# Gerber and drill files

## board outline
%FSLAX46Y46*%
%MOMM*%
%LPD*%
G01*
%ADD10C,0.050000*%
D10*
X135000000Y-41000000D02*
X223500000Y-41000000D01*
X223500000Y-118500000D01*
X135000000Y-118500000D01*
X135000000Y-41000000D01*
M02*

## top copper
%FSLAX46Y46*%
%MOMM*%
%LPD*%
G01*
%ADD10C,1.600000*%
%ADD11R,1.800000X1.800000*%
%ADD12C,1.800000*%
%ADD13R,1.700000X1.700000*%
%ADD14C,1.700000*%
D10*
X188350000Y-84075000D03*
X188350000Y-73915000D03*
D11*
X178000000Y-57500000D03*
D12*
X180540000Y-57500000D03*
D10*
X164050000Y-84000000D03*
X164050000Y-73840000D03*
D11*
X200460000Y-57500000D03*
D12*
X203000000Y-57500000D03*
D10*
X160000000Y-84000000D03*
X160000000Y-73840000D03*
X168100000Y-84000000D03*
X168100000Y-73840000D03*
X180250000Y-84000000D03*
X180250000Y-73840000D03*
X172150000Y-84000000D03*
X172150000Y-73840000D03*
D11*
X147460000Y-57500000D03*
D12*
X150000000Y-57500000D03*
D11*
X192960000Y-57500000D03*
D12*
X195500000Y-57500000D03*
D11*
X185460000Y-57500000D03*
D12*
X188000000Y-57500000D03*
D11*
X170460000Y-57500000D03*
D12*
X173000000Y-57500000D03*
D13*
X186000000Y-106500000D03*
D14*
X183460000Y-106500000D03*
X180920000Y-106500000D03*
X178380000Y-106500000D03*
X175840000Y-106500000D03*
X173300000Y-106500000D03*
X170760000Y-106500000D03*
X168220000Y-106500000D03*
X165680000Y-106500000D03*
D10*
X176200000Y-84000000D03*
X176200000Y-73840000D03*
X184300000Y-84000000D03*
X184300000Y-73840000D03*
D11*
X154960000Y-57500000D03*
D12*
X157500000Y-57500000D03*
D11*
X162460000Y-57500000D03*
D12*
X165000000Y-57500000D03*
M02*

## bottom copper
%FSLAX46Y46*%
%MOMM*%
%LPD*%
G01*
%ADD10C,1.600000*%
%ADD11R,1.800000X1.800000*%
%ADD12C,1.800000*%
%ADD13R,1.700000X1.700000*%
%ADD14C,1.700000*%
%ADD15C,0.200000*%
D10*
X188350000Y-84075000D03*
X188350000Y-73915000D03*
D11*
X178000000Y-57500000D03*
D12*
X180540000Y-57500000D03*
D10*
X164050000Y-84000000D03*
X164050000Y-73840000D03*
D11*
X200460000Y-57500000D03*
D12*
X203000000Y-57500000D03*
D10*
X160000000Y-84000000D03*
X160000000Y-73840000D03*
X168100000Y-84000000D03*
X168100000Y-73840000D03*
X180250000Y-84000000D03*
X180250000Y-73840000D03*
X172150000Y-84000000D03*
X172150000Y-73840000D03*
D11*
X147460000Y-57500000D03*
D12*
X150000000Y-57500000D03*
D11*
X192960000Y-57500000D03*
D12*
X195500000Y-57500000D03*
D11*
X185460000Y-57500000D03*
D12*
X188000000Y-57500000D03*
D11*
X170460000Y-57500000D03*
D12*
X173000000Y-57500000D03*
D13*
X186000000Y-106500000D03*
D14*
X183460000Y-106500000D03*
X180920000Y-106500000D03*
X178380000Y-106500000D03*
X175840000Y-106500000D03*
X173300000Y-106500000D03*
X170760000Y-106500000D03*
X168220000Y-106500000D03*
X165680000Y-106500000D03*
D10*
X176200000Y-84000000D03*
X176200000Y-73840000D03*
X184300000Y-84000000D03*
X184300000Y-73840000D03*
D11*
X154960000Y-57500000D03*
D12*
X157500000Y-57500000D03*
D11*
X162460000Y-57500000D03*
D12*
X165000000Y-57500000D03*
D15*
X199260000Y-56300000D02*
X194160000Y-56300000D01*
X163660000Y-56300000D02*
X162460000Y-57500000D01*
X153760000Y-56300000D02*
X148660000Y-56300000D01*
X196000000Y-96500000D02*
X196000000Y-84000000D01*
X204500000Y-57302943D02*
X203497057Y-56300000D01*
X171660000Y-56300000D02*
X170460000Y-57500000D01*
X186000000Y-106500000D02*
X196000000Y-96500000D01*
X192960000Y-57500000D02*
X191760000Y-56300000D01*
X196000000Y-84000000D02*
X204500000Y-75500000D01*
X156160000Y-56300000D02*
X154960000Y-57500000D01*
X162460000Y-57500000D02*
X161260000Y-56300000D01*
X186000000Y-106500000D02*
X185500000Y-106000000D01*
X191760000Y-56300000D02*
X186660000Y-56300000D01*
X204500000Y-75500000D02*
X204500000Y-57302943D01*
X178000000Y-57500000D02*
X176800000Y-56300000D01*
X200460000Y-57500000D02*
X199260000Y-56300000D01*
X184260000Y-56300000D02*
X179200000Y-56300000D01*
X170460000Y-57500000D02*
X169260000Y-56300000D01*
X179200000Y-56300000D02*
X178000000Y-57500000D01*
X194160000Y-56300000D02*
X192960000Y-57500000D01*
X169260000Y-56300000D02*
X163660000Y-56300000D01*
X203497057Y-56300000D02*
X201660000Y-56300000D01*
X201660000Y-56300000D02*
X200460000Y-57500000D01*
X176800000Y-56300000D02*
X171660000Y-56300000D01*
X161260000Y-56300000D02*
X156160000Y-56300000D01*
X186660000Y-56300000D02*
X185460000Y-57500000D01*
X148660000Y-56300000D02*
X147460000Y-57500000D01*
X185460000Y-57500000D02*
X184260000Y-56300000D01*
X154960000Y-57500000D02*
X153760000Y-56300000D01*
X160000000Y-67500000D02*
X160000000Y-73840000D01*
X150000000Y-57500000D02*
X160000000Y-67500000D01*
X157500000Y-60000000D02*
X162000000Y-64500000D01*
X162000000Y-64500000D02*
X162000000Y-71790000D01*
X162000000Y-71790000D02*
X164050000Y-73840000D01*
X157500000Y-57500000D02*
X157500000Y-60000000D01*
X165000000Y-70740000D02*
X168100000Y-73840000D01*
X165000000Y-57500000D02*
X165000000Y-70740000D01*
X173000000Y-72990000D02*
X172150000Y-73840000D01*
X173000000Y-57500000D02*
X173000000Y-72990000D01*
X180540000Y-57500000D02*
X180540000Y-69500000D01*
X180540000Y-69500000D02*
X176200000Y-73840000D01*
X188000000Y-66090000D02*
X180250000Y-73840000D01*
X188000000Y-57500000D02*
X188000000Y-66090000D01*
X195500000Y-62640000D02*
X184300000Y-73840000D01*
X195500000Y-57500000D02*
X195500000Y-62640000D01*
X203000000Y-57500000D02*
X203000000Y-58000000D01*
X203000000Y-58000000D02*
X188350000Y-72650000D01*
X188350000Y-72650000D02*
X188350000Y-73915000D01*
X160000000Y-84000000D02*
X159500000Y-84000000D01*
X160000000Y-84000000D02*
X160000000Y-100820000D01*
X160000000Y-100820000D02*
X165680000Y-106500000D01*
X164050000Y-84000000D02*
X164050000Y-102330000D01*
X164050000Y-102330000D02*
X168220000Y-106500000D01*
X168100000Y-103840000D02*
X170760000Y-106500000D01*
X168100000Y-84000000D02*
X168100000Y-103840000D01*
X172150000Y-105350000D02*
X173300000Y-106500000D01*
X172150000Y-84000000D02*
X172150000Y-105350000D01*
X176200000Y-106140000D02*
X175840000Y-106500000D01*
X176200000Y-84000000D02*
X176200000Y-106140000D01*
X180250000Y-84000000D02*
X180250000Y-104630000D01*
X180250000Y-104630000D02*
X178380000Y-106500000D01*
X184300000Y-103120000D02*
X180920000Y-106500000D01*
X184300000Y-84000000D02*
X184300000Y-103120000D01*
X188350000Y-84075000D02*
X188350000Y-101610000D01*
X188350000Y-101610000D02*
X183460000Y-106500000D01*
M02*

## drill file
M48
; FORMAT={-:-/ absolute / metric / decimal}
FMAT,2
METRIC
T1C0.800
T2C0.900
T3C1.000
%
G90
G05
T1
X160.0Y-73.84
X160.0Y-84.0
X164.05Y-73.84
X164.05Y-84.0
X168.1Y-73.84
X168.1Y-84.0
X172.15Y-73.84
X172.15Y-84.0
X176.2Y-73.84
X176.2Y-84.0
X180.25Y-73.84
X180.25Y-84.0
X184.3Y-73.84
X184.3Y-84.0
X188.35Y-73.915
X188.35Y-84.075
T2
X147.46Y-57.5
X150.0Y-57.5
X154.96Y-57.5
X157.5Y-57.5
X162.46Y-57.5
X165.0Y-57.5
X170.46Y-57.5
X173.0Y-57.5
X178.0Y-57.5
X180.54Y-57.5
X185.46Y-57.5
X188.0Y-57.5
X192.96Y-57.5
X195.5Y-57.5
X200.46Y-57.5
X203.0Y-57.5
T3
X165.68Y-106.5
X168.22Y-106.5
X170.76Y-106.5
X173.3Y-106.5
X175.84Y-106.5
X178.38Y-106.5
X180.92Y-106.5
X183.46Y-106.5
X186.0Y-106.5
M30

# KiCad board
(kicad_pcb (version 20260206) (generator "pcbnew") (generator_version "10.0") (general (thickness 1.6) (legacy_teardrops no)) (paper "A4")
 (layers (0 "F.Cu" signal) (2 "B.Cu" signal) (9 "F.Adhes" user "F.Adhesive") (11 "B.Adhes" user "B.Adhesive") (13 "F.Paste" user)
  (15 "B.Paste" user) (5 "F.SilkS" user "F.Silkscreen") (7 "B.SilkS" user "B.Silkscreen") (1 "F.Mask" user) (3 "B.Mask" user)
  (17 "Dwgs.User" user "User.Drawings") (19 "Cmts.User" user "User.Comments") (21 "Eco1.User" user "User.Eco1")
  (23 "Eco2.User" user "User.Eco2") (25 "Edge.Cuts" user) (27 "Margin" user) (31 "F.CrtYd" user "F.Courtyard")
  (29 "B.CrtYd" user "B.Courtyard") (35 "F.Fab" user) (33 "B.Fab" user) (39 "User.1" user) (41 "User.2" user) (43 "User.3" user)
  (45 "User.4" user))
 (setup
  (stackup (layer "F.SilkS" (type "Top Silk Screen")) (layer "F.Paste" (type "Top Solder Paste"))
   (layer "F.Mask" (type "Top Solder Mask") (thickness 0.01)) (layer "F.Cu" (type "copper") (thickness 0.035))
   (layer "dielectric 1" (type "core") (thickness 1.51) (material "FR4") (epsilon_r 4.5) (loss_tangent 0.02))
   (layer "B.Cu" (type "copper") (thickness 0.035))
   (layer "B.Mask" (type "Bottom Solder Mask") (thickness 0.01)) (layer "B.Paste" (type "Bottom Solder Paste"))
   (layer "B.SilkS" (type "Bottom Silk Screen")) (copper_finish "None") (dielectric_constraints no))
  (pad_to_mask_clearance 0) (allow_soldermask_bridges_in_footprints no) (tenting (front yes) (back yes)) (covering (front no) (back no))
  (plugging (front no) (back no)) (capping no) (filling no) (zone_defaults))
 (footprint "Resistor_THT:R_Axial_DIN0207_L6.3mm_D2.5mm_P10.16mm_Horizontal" (layer "F.Cu") (at 188.35 84.075 90)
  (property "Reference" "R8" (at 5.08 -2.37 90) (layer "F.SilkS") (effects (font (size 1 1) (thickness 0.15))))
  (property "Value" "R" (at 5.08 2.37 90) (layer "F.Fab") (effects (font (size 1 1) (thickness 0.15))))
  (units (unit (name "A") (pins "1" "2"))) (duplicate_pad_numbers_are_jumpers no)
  (pad "1" thru_hole circle (at 0 0 90) (size 1.6 1.6) (drill 0.8) (layers "*.Cu" "*.Mask") (remove_unused_layers no) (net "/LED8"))
  (pad "2" thru_hole circle (at 10.16 0 90) (size 1.6 1.6) (drill 0.8) (layers "*.Cu" "*.Mask") (remove_unused_layers no) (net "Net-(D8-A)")))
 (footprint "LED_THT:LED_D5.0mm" (layer "F.Cu") (at 178 57.5)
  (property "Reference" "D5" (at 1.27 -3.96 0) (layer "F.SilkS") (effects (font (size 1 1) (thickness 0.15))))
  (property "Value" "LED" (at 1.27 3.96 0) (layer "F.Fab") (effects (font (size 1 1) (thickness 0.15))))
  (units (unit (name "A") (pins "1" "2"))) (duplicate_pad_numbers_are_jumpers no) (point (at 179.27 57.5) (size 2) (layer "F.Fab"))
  (pad "1" thru_hole rect (at 0 0) (size 1.8 1.8) (drill 0.9) (layers "*.Cu" "*.Mask") (remove_unused_layers no) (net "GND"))
  (pad "2" thru_hole circle (at 2.54 0) (size 1.8 1.8) (drill 0.9) (layers "*.Cu" "*.Mask") (remove_unused_layers no) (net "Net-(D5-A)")))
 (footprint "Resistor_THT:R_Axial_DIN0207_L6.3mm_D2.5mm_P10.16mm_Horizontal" (layer "F.Cu") (at 164.05 84 90)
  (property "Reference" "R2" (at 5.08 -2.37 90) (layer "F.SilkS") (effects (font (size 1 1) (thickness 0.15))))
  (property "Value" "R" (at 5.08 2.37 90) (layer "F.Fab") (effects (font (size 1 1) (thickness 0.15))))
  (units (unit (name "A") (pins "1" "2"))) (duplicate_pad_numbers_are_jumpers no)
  (pad "1" thru_hole circle (at 0 0 90) (size 1.6 1.6) (drill 0.8) (layers "*.Cu" "*.Mask") (remove_unused_layers no) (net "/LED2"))
  (pad "2" thru_hole circle (at 10.16 0 90) (size 1.6 1.6) (drill 0.8) (layers "*.Cu" "*.Mask") (remove_unused_layers no) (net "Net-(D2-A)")))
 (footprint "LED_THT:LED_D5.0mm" (layer "F.Cu") (at 200.46 57.5)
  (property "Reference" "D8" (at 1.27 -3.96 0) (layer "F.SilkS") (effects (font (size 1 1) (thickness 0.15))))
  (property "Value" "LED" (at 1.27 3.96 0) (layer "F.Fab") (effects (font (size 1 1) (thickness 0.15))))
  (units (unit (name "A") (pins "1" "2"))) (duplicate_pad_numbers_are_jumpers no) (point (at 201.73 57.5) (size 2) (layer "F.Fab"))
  (pad "1" thru_hole rect (at 0 0) (size 1.8 1.8) (drill 0.9) (layers "*.Cu" "*.Mask") (remove_unused_layers no) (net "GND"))
  (pad "2" thru_hole circle (at 2.54 0) (size 1.8 1.8) (drill 0.9) (layers "*.Cu" "*.Mask") (remove_unused_layers no) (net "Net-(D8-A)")))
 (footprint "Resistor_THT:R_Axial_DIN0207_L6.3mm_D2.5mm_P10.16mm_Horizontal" (layer "F.Cu") (at 160 84 90)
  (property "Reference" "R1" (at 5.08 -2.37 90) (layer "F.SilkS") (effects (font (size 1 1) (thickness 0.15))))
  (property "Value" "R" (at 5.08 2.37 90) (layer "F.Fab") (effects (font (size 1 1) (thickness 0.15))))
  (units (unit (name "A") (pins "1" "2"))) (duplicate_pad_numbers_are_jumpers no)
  (pad "1" thru_hole circle (at 0 0 90) (size 1.6 1.6) (drill 0.8) (layers "*.Cu" "*.Mask") (remove_unused_layers no) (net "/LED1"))
  (pad "2" thru_hole circle (at 10.16 0 90) (size 1.6 1.6) (drill 0.8) (layers "*.Cu" "*.Mask") (remove_unused_layers no) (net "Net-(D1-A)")))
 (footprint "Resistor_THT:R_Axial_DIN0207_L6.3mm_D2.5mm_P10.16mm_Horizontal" (layer "F.Cu") (at 168.1 84 90)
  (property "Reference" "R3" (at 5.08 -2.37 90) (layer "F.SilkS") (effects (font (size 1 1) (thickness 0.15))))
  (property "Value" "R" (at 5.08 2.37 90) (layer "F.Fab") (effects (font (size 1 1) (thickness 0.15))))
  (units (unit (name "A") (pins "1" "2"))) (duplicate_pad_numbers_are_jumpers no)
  (pad "1" thru_hole circle (at 0 0 90) (size 1.6 1.6) (drill 0.8) (layers "*.Cu" "*.Mask") (remove_unused_layers no) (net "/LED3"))
  (pad "2" thru_hole circle (at 10.16 0 90) (size 1.6 1.6) (drill 0.8) (layers "*.Cu" "*.Mask") (remove_unused_layers no) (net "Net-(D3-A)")))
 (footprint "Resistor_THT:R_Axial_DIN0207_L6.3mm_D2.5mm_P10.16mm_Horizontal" (layer "F.Cu") (at 180.25 84 90)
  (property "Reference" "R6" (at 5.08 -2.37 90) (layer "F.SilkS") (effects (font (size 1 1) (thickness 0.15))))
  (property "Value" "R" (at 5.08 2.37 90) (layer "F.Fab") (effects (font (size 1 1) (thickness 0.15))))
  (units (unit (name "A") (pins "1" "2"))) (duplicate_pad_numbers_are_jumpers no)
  (pad "1" thru_hole circle (at 0 0 90) (size 1.6 1.6) (drill 0.8) (layers "*.Cu" "*.Mask") (remove_unused_layers no) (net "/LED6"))
  (pad "2" thru_hole circle (at 10.16 0 90) (size 1.6 1.6) (drill 0.8) (layers "*.Cu" "*.Mask") (remove_unused_layers no) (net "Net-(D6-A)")))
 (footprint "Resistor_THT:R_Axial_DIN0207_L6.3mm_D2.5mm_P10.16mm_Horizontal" (layer "F.Cu") (at 172.15 84 90)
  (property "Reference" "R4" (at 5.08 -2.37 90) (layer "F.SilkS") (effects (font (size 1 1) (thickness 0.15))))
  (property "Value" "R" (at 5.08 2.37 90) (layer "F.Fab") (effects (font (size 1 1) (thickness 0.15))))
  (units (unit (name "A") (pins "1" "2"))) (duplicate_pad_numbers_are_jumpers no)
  (pad "1" thru_hole circle (at 0 0 90) (size 1.6 1.6) (drill 0.8) (layers "*.Cu" "*.Mask") (remove_unused_layers no) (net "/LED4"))
  (pad "2" thru_hole circle (at 10.16 0 90) (size 1.6 1.6) (drill 0.8) (layers "*.Cu" "*.Mask") (remove_unused_layers no) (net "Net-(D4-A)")))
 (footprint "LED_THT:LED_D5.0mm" (layer "F.Cu") (at 147.46 57.5)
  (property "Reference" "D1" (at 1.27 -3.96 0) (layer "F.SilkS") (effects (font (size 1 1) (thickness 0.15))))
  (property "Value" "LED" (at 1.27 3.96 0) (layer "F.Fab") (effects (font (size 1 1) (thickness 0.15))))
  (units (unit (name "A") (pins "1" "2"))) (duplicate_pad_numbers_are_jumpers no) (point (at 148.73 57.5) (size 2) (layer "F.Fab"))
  (pad "1" thru_hole rect (at 0 0) (size 1.8 1.8) (drill 0.9) (layers "*.Cu" "*.Mask") (remove_unused_layers no) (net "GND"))
  (pad "2" thru_hole circle (at 2.54 0) (size 1.8 1.8) (drill 0.9) (layers "*.Cu" "*.Mask") (remove_unused_layers no) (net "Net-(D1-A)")))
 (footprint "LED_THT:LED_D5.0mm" (layer "F.Cu") (at 192.96 57.5)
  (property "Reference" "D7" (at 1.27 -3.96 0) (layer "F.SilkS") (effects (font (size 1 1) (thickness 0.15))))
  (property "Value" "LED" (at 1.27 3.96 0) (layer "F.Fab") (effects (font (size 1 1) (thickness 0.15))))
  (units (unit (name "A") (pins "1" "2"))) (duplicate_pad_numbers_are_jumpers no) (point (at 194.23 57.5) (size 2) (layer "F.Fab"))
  (pad "1" thru_hole rect (at 0 0) (size 1.8 1.8) (drill 0.9) (layers "*.Cu" "*.Mask") (remove_unused_layers no) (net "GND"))
  (pad "2" thru_hole circle (at 2.54 0) (size 1.8 1.8) (drill 0.9) (layers "*.Cu" "*.Mask") (remove_unused_layers no) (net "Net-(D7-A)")))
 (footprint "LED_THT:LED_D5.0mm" (layer "F.Cu") (at 185.46 57.5)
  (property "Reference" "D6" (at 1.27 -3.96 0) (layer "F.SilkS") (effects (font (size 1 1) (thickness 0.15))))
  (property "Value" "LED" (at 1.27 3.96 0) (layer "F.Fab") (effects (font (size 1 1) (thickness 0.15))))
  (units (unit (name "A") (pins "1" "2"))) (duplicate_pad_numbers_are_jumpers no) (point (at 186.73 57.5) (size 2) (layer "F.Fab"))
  (pad "1" thru_hole rect (at 0 0) (size 1.8 1.8) (drill 0.9) (layers "*.Cu" "*.Mask") (remove_unused_layers no) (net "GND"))
  (pad "2" thru_hole circle (at 2.54 0) (size 1.8 1.8) (drill 0.9) (layers "*.Cu" "*.Mask") (remove_unused_layers no) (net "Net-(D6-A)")))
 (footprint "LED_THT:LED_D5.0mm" (layer "F.Cu") (at 170.46 57.5)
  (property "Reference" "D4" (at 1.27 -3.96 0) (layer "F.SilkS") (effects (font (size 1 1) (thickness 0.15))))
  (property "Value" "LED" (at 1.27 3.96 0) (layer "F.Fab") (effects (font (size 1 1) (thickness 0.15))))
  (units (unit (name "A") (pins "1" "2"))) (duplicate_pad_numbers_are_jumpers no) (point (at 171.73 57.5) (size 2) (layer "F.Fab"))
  (pad "1" thru_hole rect (at 0 0) (size 1.8 1.8) (drill 0.9) (layers "*.Cu" "*.Mask") (remove_unused_layers no) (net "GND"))
  (pad "2" thru_hole circle (at 2.54 0) (size 1.8 1.8) (drill 0.9) (layers "*.Cu" "*.Mask") (remove_unused_layers no) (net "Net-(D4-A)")))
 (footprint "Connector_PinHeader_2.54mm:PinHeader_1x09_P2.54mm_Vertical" (layer "F.Cu") (at 186 106.5 -90)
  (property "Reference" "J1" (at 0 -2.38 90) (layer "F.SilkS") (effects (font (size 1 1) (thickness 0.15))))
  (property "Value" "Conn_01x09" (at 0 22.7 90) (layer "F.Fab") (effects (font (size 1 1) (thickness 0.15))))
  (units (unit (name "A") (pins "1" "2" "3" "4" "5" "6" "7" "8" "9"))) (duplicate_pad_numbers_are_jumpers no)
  (pad "1" thru_hole rect (at 0 0 270) (size 1.7 1.7) (drill 1) (layers "*.Cu" "*.Mask") (remove_unused_layers no) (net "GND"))
  (pad "2" thru_hole circle (at 0 2.54 270) (size 1.7 1.7) (drill 1) (layers "*.Cu" "*.Mask") (remove_unused_layers no) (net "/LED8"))
  (pad "3" thru_hole circle (at 0 5.08 270) (size 1.7 1.7) (drill 1) (layers "*.Cu" "*.Mask") (remove_unused_layers no) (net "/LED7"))
  (pad "4" thru_hole circle (at 0 7.62 270) (size 1.7 1.7) (drill 1) (layers "*.Cu" "*.Mask") (remove_unused_layers no) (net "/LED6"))
  (pad "5" thru_hole circle (at 0 10.16 270) (size 1.7 1.7) (drill 1) (layers "*.Cu" "*.Mask") (remove_unused_layers no) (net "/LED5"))
  (pad "6" thru_hole circle (at 0 12.7 270) (size 1.7 1.7) (drill 1) (layers "*.Cu" "*.Mask") (remove_unused_layers no) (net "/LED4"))
  (pad "7" thru_hole circle (at 0 15.24 270) (size 1.7 1.7) (drill 1) (layers "*.Cu" "*.Mask") (remove_unused_layers no) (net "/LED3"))
  (pad "8" thru_hole circle (at 0 17.78 270) (size 1.7 1.7) (drill 1) (layers "*.Cu" "*.Mask") (remove_unused_layers no) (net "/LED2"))
  (pad "9" thru_hole circle (at 0 20.32 270) (size 1.7 1.7) (drill 1) (layers "*.Cu" "*.Mask") (remove_unused_layers no) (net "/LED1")))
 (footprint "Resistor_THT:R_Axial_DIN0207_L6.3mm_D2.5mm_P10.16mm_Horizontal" (layer "F.Cu") (at 176.2 84 90)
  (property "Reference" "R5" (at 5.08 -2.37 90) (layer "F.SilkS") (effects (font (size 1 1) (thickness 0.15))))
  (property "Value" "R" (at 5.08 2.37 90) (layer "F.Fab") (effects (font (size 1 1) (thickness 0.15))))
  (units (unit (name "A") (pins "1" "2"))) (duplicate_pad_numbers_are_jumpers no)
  (pad "1" thru_hole circle (at 0 0 90) (size 1.6 1.6) (drill 0.8) (layers "*.Cu" "*.Mask") (remove_unused_layers no) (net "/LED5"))
  (pad "2" thru_hole circle (at 10.16 0 90) (size 1.6 1.6) (drill 0.8) (layers "*.Cu" "*.Mask") (remove_unused_layers no) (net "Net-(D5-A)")))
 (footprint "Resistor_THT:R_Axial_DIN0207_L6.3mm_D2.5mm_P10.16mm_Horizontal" (layer "F.Cu") (at 184.3 84 90)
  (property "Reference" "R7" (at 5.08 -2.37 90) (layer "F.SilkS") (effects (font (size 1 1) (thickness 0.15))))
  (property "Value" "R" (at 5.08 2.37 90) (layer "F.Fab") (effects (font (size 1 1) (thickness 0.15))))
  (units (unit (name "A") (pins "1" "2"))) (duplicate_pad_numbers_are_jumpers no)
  (pad "1" thru_hole circle (at 0 0 90) (size 1.6 1.6) (drill 0.8) (layers "*.Cu" "*.Mask") (remove_unused_layers no) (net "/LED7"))
  (pad "2" thru_hole circle (at 10.16 0 90) (size 1.6 1.6) (drill 0.8) (layers "*.Cu" "*.Mask") (remove_unused_layers no) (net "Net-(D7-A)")))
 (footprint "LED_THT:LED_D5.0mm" (layer "F.Cu") (at 154.96 57.5)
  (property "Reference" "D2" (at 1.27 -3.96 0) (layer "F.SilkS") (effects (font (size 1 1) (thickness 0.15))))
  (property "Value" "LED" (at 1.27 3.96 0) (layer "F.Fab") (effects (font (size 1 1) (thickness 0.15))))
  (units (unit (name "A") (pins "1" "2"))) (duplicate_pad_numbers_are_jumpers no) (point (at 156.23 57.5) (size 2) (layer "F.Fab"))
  (pad "1" thru_hole rect (at 0 0) (size 1.8 1.8) (drill 0.9) (layers "*.Cu" "*.Mask") (remove_unused_layers no) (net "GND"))
  (pad "2" thru_hole circle (at 2.54 0) (size 1.8 1.8) (drill 0.9) (layers "*.Cu" "*.Mask") (remove_unused_layers no) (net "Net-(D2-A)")))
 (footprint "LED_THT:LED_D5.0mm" (layer "F.Cu") (at 162.46 57.5)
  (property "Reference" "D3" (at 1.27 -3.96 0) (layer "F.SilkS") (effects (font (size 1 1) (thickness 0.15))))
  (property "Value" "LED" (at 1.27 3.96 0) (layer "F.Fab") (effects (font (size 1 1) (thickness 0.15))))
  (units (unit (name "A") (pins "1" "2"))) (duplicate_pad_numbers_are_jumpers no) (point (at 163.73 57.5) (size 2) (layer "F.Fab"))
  (pad "1" thru_hole rect (at 0 0) (size 1.8 1.8) (drill 0.9) (layers "*.Cu" "*.Mask") (remove_unused_layers no) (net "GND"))
  (pad "2" thru_hole circle (at 2.54 0) (size 1.8 1.8) (drill 0.9) (layers "*.Cu" "*.Mask") (remove_unused_layers no) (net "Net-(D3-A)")))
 (gr_rect (start 135 41) (end 223.5 118.5) (stroke (width 0.05) (type default)) (fill no) (layer "Edge.Cuts"))
 (segment (start 199.26 56.3) (end 194.16 56.3) (width 0.2) (layer "B.Cu") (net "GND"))
 (segment (start 163.66 56.3) (end 162.46 57.5) (width 0.2) (layer "B.Cu") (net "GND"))
 (segment (start 153.76 56.3) (end 148.66 56.3) (width 0.2) (layer "B.Cu") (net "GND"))
 (segment (start 196 96.5) (end 196 84) (width 0.2) (layer "B.Cu") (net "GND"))
 (segment (start 204.5 57.302943) (end 203.497057 56.3) (width 0.2) (layer "B.Cu") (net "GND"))
 (segment (start 171.66 56.3) (end 170.46 57.5) (width 0.2) (layer "B.Cu") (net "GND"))
 (segment (start 186 106.5) (end 196 96.5) (width 0.2) (layer "B.Cu") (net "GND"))
 (segment (start 192.96 57.5) (end 191.76 56.3) (width 0.2) (layer "B.Cu") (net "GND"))
 (segment (start 196 84) (end 204.5 75.5) (width 0.2) (layer "B.Cu") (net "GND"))
 (segment (start 156.16 56.3) (end 154.96 57.5) (width 0.2) (layer "B.Cu") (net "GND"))
 (segment (start 162.46 57.5) (end 161.26 56.3) (width 0.2) (layer "B.Cu") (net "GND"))
 (segment (start 186 106.5) (end 185.5 106) (width 0.2) (layer "B.Cu") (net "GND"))
 (segment (start 191.76 56.3) (end 186.66 56.3) (width 0.2) (layer "B.Cu") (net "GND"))
 (segment (start 204.5 75.5) (end 204.5 57.302943) (width 0.2) (layer "B.Cu") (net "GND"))
 (segment (start 178 57.5) (end 176.8 56.3) (width 0.2) (layer "B.Cu") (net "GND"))
 (segment (start 200.46 57.5) (end 199.26 56.3) (width 0.2) (layer "B.Cu") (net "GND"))
 (segment (start 184.26 56.3) (end 179.2 56.3) (width 0.2) (layer "B.Cu") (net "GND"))
 (segment (start 170.46 57.5) (end 169.26 56.3) (width 0.2) (layer "B.Cu") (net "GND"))
 (segment (start 179.2 56.3) (end 178 57.5) (width 0.2) (layer "B.Cu") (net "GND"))
 (segment (start 194.16 56.3) (end 192.96 57.5) (width 0.2) (layer "B.Cu") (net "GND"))
 (segment (start 169.26 56.3) (end 163.66 56.3) (width 0.2) (layer "B.Cu") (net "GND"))
 (segment (start 203.497057 56.3) (end 201.66 56.3) (width 0.2) (layer "B.Cu") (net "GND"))
 (segment (start 201.66 56.3) (end 200.46 57.5) (width 0.2) (layer "B.Cu") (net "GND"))
 (segment (start 176.8 56.3) (end 171.66 56.3) (width 0.2) (layer "B.Cu") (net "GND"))
 (segment (start 161.26 56.3) (end 156.16 56.3) (width 0.2) (layer "B.Cu") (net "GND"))
 (segment (start 186.66 56.3) (end 185.46 57.5) (width 0.2) (layer "B.Cu") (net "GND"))
 (segment (start 148.66 56.3) (end 147.46 57.5) (width 0.2) (layer "B.Cu") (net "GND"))
 (segment (start 185.46 57.5) (end 184.26 56.3) (width 0.2) (layer "B.Cu") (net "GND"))
 (segment (start 154.96 57.5) (end 153.76 56.3) (width 0.2) (layer "B.Cu") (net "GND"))
 (segment (start 160 67.5) (end 160 73.84) (width 0.2) (layer "B.Cu") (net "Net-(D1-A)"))
 (segment (start 150 57.5) (end 160 67.5) (width 0.2) (layer "B.Cu") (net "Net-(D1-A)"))
 (segment (start 157.5 60) (end 162 64.5) (width 0.2) (layer "B.Cu") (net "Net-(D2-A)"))
 (segment (start 162 64.5) (end 162 71.79) (width 0.2) (layer "B.Cu") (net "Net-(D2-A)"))
 (segment (start 162 71.79) (end 164.05 73.84) (width 0.2) (layer "B.Cu") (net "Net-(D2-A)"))
 (segment (start 157.5 57.5) (end 157.5 60) (width 0.2) (layer "B.Cu") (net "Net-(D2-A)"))
 (segment (start 165 70.74) (end 168.1 73.84) (width 0.2) (layer "B.Cu") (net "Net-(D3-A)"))
 (segment (start 165 57.5) (end 165 70.74) (width 0.2) (layer "B.Cu") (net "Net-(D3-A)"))
 (segment (start 173 72.99) (end 172.15 73.84) (width 0.2) (layer "B.Cu") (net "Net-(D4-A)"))
 (segment (start 173 57.5) (end 173 72.99) (width 0.2) (layer "B.Cu") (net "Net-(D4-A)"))
 (segment (start 180.54 57.5) (end 180.54 69.5) (width 0.2) (layer "B.Cu") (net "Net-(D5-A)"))
 (segment (start 180.54 69.5) (end 176.2 73.84) (width 0.2) (layer "B.Cu") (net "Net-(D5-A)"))
 (segment (start 188 66.09) (end 180.25 73.84) (width 0.2) (layer "B.Cu") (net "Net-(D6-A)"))
 (segment (start 188 57.5) (end 188 66.09) (width 0.2) (layer "B.Cu") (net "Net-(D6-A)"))
 (segment (start 195.5 62.64) (end 184.3 73.84) (width 0.2) (layer "B.Cu") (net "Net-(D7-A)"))
 (segment (start 195.5 57.5) (end 195.5 62.64) (width 0.2) (layer "B.Cu") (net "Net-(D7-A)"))
 (segment (start 203 57.5) (end 203 58) (width 0.2) (layer "B.Cu") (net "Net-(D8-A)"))
 (segment (start 203 58) (end 188.35 72.65) (width 0.2) (layer "B.Cu") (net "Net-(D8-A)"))
 (segment (start 188.35 72.65) (end 188.35 73.915) (width 0.2) (layer "B.Cu") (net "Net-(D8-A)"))
 (segment (start 160 84) (end 159.5 84) (width 0.2) (layer "B.Cu") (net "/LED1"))
 (segment (start 160 84) (end 160 100.82) (width 0.2) (layer "B.Cu") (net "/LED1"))
 (segment (start 160 100.82) (end 165.68 106.5) (width 0.2) (layer "B.Cu") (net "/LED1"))
 (segment (start 164.05 84) (end 164.05 102.33) (width 0.2) (layer "B.Cu") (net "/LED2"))
 (segment (start 164.05 102.33) (end 168.22 106.5) (width 0.2) (layer "B.Cu") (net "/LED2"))
 (segment (start 168.1 103.84) (end 170.76 106.5) (width 0.2) (layer "B.Cu") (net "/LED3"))
 (segment (start 168.1 84) (end 168.1 103.84) (width 0.2) (layer "B.Cu") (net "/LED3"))
 (segment (start 172.15 105.35) (end 173.3 106.5) (width 0.2) (layer "B.Cu") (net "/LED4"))
 (segment (start 172.15 84) (end 172.15 105.35) (width 0.2) (layer "B.Cu") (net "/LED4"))
 (segment (start 176.2 106.14) (end 175.84 106.5) (width 0.2) (layer "B.Cu") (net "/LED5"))
 (segment (start 176.2 84) (end 176.2 106.14) (width 0.2) (layer "B.Cu") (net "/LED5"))
 (segment (start 180.25 84) (end 180.25 104.63) (width 0.2) (layer "B.Cu") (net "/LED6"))
 (segment (start 180.25 104.63) (end 178.38 106.5) (width 0.2) (layer "B.Cu") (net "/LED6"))
 (segment (start 184.3 103.12) (end 180.92 106.5) (width 0.2) (layer "B.Cu") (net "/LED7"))
 (segment (start 184.3 84) (end 184.3 103.12) (width 0.2) (layer "B.Cu") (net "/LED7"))
 (segment (start 188.35 84.075) (end 188.35 101.61) (width 0.2) (layer "B.Cu") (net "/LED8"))
 (segment (start 188.35 101.61) (end 183.46 106.5) (width 0.2) (layer "B.Cu") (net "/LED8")))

